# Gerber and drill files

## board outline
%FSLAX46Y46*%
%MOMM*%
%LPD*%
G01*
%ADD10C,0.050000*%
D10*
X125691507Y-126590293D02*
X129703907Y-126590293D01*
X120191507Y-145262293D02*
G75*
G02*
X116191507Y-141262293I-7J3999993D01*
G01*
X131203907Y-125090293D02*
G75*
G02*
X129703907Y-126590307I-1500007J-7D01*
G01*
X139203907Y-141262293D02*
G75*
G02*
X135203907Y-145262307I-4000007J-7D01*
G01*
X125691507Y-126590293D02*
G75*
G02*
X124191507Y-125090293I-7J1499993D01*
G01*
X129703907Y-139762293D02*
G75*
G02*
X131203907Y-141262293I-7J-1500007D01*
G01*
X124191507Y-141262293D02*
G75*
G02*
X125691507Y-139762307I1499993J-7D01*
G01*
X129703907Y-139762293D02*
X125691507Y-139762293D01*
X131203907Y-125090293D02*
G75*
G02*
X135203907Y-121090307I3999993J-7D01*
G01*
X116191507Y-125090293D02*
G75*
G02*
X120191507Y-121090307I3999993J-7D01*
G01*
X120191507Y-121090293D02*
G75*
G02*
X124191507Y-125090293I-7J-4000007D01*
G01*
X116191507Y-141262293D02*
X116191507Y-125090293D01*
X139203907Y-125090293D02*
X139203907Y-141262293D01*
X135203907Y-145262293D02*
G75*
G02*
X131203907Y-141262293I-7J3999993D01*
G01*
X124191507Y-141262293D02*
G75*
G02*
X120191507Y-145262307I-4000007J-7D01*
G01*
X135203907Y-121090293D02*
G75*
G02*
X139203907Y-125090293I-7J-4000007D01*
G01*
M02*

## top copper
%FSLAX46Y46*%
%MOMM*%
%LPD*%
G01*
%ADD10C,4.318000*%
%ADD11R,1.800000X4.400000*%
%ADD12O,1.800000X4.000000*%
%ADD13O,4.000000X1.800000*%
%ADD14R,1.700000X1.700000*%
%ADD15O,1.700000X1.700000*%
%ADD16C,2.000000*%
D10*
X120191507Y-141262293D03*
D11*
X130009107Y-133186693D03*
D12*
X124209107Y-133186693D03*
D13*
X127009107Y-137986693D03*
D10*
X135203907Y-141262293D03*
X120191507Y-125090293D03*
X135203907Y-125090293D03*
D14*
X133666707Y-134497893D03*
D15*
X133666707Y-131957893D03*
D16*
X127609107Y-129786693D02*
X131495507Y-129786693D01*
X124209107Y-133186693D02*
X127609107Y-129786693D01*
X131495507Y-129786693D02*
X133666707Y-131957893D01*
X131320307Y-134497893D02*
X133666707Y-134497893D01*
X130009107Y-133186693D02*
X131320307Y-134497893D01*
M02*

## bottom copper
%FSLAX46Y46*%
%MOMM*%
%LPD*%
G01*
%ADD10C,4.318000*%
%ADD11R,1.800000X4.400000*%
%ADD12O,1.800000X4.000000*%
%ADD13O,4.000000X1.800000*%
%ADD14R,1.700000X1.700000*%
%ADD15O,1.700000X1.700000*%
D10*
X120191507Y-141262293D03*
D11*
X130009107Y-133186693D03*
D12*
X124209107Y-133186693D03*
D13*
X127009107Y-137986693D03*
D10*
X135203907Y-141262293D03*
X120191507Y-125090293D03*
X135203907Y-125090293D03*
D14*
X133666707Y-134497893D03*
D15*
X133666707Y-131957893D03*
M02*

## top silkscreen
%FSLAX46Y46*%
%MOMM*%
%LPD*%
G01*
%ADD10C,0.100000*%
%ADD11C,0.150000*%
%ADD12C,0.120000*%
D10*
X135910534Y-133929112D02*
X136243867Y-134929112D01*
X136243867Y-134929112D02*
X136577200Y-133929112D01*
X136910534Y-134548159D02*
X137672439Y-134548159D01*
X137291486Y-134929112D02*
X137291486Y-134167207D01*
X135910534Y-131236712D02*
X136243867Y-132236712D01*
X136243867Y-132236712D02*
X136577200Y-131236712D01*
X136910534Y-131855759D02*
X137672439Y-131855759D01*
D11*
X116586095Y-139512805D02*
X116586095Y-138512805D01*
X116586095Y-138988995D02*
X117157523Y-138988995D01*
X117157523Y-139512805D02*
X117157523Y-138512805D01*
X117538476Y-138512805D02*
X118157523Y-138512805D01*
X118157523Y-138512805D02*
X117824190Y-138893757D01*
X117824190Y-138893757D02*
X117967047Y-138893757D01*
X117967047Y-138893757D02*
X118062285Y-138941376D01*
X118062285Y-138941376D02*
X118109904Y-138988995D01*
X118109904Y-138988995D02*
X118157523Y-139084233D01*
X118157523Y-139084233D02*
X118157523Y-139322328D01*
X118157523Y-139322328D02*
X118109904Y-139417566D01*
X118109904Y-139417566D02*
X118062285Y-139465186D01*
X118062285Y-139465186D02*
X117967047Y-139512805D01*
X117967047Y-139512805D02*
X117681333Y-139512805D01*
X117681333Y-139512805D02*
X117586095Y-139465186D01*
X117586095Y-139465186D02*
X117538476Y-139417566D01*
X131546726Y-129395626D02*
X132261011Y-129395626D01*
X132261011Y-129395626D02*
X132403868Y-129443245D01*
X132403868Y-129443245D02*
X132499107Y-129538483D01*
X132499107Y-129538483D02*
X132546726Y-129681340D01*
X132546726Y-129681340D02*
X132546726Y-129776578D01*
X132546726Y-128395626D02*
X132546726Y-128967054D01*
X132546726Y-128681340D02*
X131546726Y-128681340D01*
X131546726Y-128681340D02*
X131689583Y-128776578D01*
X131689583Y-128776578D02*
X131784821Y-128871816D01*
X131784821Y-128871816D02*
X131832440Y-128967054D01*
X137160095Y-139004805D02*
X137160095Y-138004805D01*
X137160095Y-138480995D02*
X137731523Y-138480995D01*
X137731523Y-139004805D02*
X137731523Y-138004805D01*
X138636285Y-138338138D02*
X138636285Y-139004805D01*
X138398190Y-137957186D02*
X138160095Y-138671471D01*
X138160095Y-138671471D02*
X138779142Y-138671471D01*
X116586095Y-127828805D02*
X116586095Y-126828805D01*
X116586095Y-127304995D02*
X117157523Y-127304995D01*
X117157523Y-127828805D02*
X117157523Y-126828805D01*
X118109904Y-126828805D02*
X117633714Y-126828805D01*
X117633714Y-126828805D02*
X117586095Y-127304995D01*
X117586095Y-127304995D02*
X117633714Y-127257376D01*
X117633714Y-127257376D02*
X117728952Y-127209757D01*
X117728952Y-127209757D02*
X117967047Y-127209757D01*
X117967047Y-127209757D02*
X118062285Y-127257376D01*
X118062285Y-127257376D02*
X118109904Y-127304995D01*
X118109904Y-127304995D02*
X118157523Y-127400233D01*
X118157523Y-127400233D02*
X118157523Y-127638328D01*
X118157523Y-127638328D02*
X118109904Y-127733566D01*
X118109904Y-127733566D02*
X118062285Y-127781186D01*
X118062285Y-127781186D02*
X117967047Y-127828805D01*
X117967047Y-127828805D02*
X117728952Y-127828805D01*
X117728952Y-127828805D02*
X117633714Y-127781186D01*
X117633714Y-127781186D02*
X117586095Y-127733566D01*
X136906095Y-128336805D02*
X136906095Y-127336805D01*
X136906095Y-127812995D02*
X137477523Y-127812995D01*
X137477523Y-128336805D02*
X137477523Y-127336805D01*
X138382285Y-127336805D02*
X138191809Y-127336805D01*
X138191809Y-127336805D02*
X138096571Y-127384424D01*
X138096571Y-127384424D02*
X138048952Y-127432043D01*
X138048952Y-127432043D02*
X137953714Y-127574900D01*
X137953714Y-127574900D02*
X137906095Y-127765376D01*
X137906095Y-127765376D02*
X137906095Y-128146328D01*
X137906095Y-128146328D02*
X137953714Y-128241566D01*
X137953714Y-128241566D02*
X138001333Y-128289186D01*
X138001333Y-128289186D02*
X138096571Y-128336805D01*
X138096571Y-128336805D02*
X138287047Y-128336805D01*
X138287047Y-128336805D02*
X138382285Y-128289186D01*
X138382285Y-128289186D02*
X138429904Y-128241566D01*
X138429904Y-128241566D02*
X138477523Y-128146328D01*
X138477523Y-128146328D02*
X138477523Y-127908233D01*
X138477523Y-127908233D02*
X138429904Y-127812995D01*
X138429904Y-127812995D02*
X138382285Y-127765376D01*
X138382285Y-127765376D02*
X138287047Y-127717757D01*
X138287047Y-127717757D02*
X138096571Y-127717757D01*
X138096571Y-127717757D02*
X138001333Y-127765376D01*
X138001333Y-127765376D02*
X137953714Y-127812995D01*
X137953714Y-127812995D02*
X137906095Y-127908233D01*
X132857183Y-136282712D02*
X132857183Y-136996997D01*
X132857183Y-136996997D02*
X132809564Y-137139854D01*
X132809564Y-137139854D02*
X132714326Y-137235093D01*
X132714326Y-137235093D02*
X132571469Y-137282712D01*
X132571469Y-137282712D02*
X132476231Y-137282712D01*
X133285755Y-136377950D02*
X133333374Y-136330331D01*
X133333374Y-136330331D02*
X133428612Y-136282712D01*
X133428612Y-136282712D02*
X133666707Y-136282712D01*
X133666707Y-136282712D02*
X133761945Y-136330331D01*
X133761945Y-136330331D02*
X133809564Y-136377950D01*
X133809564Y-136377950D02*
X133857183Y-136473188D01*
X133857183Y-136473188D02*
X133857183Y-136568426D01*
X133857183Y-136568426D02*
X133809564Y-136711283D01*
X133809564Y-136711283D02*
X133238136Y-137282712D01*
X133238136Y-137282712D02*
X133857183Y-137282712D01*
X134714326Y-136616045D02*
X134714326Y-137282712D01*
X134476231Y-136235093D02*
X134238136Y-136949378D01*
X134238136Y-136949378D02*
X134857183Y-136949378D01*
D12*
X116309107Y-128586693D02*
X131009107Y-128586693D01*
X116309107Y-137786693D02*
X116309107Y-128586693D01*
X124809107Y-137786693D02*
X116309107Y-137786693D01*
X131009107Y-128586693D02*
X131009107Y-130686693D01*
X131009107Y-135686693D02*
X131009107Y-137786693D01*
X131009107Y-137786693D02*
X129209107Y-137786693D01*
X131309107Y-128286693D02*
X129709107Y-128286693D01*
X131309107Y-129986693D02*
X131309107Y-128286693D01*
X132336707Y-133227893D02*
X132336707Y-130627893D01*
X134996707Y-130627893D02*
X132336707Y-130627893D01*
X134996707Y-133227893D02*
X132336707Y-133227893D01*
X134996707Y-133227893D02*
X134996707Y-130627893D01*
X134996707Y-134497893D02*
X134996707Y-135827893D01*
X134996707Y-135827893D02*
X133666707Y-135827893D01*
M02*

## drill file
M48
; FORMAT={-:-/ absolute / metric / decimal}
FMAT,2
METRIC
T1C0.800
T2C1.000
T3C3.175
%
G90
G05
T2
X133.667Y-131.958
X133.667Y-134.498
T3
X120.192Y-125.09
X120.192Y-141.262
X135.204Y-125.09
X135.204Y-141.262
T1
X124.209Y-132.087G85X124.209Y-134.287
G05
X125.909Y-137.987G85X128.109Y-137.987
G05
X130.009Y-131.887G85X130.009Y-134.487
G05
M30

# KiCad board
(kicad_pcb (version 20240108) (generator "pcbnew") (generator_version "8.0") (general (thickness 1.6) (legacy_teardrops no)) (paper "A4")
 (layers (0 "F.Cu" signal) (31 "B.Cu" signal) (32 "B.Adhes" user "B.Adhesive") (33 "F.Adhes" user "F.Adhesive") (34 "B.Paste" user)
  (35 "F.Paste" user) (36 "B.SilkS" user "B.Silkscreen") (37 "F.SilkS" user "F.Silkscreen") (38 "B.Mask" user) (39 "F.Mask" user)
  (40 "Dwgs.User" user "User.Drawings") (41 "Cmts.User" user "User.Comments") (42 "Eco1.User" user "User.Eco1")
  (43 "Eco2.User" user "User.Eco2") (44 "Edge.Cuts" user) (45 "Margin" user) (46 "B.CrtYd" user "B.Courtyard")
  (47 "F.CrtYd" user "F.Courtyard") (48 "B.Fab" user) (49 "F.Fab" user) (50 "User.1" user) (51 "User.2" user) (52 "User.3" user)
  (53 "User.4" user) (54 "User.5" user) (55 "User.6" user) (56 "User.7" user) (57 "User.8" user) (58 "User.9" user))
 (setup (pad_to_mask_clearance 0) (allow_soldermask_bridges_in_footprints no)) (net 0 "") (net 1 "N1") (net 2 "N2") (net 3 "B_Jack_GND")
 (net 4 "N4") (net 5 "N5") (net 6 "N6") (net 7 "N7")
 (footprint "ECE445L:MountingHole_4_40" (layer "F.Cu") (at 120.191507 141.262293)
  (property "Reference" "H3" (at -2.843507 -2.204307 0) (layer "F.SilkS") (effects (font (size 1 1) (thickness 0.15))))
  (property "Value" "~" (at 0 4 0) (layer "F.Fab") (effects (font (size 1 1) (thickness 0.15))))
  (pad "1" thru_hole circle (at 0 0) (size 4.318 4.318) (drill 3.175) (layers "*.Cu" "*.Mask") (remove_unused_layers no) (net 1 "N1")))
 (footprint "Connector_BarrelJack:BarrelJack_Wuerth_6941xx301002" (layer "F.Cu") (at 130.009107 133.186693 -90)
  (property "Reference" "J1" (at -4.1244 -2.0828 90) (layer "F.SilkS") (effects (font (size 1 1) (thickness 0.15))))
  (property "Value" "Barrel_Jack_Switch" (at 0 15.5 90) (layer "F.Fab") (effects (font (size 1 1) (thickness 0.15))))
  (fp_line (start -4.6 13.7) (end -4.6 -1) (stroke (width 0.12) (type solid)) (layer "F.SilkS"))
  (fp_line (start 4.6 13.7) (end -4.6 13.7) (stroke (width 0.12) (type solid)) (layer "F.SilkS"))
  (fp_line (start 4.6 5.2) (end 4.6 13.7) (stroke (width 0.12) (type solid)) (layer "F.SilkS"))
  (fp_line (start -4.6 -1) (end -2.5 -1) (stroke (width 0.12) (type solid)) (layer "F.SilkS"))
  (fp_line (start 2.5 -1) (end 4.6 -1) (stroke (width 0.12) (type solid)) (layer "F.SilkS"))
  (fp_line (start 4.6 -1) (end 4.6 0.8) (stroke (width 0.12) (type solid)) (layer "F.SilkS"))
  (fp_line (start -4.9 -1.3) (end -4.9 0.3) (stroke (width 0.12) (type solid)) (layer "F.SilkS"))
  (fp_line (start -3.2 -1.3) (end -4.9 -1.3) (stroke (width 0.12) (type solid)) (layer "F.SilkS"))
  (pad "1" thru_hole rect (at 0 0 270) (size 4.4 1.8) (drill oval 3.4 0.8) (layers "*.Cu" "*.Mask") (remove_unused_layers no) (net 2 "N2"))
  (pad "2" thru_hole oval (at 0 5.8 270) (size 4 1.8) (drill oval 3 0.8) (layers "*.Cu" "*.Mask") (remove_unused_layers no)
   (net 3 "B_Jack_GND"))
  (pad "3" thru_hole oval (at 4.8 3) (size 4 1.8) (drill oval 3 0.8) (layers "*.Cu" "*.Mask") (remove_unused_layers no) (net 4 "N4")))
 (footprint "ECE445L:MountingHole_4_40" (layer "F.Cu") (at 135.203907 141.262293)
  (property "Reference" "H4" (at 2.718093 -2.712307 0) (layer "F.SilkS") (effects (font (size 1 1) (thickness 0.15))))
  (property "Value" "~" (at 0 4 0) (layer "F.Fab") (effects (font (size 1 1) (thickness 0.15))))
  (pad "1" thru_hole circle (at 0 0) (size 4.318 4.318) (drill 3.175) (layers "*.Cu" "*.Mask") (remove_unused_layers no) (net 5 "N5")))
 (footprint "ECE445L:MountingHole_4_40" (layer "F.Cu") (at 120.191507 125.090293)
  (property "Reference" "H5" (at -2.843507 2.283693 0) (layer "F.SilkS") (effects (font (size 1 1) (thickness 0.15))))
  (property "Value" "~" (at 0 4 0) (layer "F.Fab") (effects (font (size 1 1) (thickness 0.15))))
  (pad "1" thru_hole circle (at 0 0) (size 4.318 4.318) (drill 3.175) (layers "*.Cu" "*.Mask") (remove_unused_layers no) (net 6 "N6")))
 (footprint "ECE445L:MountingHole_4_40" (layer "F.Cu") (at 135.203907 125.090293)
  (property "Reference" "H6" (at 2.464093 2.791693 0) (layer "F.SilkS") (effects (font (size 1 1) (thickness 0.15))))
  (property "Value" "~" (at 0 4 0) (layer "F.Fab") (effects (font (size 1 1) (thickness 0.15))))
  (pad "1" thru_hole circle (at 0 0) (size 4.318 4.318) (drill 3.175) (layers "*.Cu" "*.Mask") (remove_unused_layers no) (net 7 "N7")))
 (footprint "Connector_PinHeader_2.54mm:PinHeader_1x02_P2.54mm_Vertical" (layer "F.Cu") (at 133.666707 134.497893 180)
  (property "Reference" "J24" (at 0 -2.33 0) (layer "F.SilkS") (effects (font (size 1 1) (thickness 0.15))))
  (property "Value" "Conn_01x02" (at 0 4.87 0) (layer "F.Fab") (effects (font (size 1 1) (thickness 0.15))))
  (fp_line (start 1.33 1.27) (end 1.33 3.87) (stroke (width 0.12) (type solid)) (layer "F.SilkS"))
  (fp_line (start -1.33 3.87) (end 1.33 3.87) (stroke (width 0.12) (type solid)) (layer "F.SilkS"))
  (fp_line (start -1.33 1.27) (end 1.33 1.27) (stroke (width 0.12) (type solid)) (layer "F.SilkS"))
  (fp_line (start -1.33 1.27) (end -1.33 3.87) (stroke (width 0.12) (type solid)) (layer "F.SilkS"))
  (fp_line (start -1.33 0) (end -1.33 -1.33) (stroke (width 0.12) (type solid)) (layer "F.SilkS"))
  (fp_line (start -1.33 -1.33) (end 0 -1.33) (stroke (width 0.12) (type solid)) (layer "F.SilkS"))
  (pad "1" thru_hole rect (at 0 0 180) (size 1.7 1.7) (drill 1) (layers "*.Cu" "*.Mask") (remove_unused_layers no) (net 2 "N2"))
  (pad "2" thru_hole oval (at 0 2.54 180) (size 1.7 1.7) (drill 1) (layers "*.Cu" "*.Mask") (remove_unused_layers no) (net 3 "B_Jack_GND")))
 (gr_line (start 125.691507 126.590293) (end 129.703907 126.590293) (stroke (width 0.05) (type default)) (layer "Edge.Cuts"))
 (gr_arc (start 120.191507 145.262293) (mid 117.363073 144.090723) (end 116.191507 141.262293) (stroke (width 0.05) (type default))
  (layer "Edge.Cuts"))
 (gr_arc (start 131.203907 125.090293) (mid 130.764565 126.150951) (end 129.703907 126.590293) (stroke (width 0.05) (type default))
  (layer "Edge.Cuts"))
 (gr_arc (start 139.203907 141.262293) (mid 138.032332 144.090718) (end 135.203907 145.262293) (stroke (width 0.05) (type default))
  (layer "Edge.Cuts"))
 (gr_arc (start 125.691507 126.590293) (mid 124.63084 126.150956) (end 124.191507 125.090293) (stroke (width 0.05) (type default))
  (layer "Edge.Cuts"))
 (gr_arc (start 129.703907 139.762293) (mid 130.76456 140.201636) (end 131.203907 141.262293) (stroke (width 0.05) (type default))
  (layer "Edge.Cuts"))
 (gr_arc (start 124.191507 141.262293) (mid 124.630845 140.201631) (end 125.691507 139.762293) (stroke (width 0.05) (type default))
  (layer "Edge.Cuts"))
 (gr_line (start 129.703907 139.762293) (end 125.691507 139.762293) (stroke (width 0.05) (type default)) (layer "Edge.Cuts"))
 (gr_arc (start 131.203907 125.090293) (mid 132.375478 122.261864) (end 135.203907 121.090293) (stroke (width 0.05) (type default))
  (layer "Edge.Cuts"))
 (gr_arc (start 116.191507 125.090293) (mid 117.363078 122.261864) (end 120.191507 121.090293) (stroke (width 0.05) (type default))
  (layer "Edge.Cuts"))
 (gr_arc (start 120.191507 121.090293) (mid 123.019927 122.261869) (end 124.191507 125.090293) (stroke (width 0.05) (type default))
  (layer "Edge.Cuts"))
 (gr_line (start 116.191507 141.262293) (end 116.191507 125.090293) (stroke (width 0.05) (type default)) (layer "Edge.Cuts"))
 (gr_line (start 139.203907 125.090293) (end 139.203907 141.262293) (stroke (width 0.05) (type default)) (layer "Edge.Cuts"))
 (gr_arc (start 135.203907 145.262293) (mid 132.375473 144.090723) (end 131.203907 141.262293) (stroke (width 0.05) (type default))
  (layer "Edge.Cuts"))
 (gr_arc (start 124.191507 141.262293) (mid 123.019932 144.090718) (end 120.191507 145.262293) (stroke (width 0.05) (type default))
  (layer "Edge.Cuts"))
 (gr_arc (start 135.203907 121.090293) (mid 138.032327 122.261869) (end 139.203907 125.090293) (stroke (width 0.05) (type default))
  (layer "Edge.Cuts"))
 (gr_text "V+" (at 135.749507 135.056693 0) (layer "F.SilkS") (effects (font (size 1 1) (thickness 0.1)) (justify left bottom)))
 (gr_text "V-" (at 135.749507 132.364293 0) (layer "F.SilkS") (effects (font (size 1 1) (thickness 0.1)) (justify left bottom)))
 (segment (start 127.609107 129.786693) (end 131.495507 129.786693) (width 2) (layer "F.Cu") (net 3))
 (segment (start 124.209107 133.186693) (end 127.609107 129.786693) (width 2) (layer "F.Cu") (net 3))
 (segment (start 131.495507 129.786693) (end 133.666707 131.957893) (width 2) (layer "F.Cu") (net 3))
 (segment (start 131.320307 134.497893) (end 133.666707 134.497893) (width 2) (layer "F.Cu") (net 2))
 (segment (start 130.009107 133.186693) (end 131.320307 134.497893) (width 2) (layer "F.Cu") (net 2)))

